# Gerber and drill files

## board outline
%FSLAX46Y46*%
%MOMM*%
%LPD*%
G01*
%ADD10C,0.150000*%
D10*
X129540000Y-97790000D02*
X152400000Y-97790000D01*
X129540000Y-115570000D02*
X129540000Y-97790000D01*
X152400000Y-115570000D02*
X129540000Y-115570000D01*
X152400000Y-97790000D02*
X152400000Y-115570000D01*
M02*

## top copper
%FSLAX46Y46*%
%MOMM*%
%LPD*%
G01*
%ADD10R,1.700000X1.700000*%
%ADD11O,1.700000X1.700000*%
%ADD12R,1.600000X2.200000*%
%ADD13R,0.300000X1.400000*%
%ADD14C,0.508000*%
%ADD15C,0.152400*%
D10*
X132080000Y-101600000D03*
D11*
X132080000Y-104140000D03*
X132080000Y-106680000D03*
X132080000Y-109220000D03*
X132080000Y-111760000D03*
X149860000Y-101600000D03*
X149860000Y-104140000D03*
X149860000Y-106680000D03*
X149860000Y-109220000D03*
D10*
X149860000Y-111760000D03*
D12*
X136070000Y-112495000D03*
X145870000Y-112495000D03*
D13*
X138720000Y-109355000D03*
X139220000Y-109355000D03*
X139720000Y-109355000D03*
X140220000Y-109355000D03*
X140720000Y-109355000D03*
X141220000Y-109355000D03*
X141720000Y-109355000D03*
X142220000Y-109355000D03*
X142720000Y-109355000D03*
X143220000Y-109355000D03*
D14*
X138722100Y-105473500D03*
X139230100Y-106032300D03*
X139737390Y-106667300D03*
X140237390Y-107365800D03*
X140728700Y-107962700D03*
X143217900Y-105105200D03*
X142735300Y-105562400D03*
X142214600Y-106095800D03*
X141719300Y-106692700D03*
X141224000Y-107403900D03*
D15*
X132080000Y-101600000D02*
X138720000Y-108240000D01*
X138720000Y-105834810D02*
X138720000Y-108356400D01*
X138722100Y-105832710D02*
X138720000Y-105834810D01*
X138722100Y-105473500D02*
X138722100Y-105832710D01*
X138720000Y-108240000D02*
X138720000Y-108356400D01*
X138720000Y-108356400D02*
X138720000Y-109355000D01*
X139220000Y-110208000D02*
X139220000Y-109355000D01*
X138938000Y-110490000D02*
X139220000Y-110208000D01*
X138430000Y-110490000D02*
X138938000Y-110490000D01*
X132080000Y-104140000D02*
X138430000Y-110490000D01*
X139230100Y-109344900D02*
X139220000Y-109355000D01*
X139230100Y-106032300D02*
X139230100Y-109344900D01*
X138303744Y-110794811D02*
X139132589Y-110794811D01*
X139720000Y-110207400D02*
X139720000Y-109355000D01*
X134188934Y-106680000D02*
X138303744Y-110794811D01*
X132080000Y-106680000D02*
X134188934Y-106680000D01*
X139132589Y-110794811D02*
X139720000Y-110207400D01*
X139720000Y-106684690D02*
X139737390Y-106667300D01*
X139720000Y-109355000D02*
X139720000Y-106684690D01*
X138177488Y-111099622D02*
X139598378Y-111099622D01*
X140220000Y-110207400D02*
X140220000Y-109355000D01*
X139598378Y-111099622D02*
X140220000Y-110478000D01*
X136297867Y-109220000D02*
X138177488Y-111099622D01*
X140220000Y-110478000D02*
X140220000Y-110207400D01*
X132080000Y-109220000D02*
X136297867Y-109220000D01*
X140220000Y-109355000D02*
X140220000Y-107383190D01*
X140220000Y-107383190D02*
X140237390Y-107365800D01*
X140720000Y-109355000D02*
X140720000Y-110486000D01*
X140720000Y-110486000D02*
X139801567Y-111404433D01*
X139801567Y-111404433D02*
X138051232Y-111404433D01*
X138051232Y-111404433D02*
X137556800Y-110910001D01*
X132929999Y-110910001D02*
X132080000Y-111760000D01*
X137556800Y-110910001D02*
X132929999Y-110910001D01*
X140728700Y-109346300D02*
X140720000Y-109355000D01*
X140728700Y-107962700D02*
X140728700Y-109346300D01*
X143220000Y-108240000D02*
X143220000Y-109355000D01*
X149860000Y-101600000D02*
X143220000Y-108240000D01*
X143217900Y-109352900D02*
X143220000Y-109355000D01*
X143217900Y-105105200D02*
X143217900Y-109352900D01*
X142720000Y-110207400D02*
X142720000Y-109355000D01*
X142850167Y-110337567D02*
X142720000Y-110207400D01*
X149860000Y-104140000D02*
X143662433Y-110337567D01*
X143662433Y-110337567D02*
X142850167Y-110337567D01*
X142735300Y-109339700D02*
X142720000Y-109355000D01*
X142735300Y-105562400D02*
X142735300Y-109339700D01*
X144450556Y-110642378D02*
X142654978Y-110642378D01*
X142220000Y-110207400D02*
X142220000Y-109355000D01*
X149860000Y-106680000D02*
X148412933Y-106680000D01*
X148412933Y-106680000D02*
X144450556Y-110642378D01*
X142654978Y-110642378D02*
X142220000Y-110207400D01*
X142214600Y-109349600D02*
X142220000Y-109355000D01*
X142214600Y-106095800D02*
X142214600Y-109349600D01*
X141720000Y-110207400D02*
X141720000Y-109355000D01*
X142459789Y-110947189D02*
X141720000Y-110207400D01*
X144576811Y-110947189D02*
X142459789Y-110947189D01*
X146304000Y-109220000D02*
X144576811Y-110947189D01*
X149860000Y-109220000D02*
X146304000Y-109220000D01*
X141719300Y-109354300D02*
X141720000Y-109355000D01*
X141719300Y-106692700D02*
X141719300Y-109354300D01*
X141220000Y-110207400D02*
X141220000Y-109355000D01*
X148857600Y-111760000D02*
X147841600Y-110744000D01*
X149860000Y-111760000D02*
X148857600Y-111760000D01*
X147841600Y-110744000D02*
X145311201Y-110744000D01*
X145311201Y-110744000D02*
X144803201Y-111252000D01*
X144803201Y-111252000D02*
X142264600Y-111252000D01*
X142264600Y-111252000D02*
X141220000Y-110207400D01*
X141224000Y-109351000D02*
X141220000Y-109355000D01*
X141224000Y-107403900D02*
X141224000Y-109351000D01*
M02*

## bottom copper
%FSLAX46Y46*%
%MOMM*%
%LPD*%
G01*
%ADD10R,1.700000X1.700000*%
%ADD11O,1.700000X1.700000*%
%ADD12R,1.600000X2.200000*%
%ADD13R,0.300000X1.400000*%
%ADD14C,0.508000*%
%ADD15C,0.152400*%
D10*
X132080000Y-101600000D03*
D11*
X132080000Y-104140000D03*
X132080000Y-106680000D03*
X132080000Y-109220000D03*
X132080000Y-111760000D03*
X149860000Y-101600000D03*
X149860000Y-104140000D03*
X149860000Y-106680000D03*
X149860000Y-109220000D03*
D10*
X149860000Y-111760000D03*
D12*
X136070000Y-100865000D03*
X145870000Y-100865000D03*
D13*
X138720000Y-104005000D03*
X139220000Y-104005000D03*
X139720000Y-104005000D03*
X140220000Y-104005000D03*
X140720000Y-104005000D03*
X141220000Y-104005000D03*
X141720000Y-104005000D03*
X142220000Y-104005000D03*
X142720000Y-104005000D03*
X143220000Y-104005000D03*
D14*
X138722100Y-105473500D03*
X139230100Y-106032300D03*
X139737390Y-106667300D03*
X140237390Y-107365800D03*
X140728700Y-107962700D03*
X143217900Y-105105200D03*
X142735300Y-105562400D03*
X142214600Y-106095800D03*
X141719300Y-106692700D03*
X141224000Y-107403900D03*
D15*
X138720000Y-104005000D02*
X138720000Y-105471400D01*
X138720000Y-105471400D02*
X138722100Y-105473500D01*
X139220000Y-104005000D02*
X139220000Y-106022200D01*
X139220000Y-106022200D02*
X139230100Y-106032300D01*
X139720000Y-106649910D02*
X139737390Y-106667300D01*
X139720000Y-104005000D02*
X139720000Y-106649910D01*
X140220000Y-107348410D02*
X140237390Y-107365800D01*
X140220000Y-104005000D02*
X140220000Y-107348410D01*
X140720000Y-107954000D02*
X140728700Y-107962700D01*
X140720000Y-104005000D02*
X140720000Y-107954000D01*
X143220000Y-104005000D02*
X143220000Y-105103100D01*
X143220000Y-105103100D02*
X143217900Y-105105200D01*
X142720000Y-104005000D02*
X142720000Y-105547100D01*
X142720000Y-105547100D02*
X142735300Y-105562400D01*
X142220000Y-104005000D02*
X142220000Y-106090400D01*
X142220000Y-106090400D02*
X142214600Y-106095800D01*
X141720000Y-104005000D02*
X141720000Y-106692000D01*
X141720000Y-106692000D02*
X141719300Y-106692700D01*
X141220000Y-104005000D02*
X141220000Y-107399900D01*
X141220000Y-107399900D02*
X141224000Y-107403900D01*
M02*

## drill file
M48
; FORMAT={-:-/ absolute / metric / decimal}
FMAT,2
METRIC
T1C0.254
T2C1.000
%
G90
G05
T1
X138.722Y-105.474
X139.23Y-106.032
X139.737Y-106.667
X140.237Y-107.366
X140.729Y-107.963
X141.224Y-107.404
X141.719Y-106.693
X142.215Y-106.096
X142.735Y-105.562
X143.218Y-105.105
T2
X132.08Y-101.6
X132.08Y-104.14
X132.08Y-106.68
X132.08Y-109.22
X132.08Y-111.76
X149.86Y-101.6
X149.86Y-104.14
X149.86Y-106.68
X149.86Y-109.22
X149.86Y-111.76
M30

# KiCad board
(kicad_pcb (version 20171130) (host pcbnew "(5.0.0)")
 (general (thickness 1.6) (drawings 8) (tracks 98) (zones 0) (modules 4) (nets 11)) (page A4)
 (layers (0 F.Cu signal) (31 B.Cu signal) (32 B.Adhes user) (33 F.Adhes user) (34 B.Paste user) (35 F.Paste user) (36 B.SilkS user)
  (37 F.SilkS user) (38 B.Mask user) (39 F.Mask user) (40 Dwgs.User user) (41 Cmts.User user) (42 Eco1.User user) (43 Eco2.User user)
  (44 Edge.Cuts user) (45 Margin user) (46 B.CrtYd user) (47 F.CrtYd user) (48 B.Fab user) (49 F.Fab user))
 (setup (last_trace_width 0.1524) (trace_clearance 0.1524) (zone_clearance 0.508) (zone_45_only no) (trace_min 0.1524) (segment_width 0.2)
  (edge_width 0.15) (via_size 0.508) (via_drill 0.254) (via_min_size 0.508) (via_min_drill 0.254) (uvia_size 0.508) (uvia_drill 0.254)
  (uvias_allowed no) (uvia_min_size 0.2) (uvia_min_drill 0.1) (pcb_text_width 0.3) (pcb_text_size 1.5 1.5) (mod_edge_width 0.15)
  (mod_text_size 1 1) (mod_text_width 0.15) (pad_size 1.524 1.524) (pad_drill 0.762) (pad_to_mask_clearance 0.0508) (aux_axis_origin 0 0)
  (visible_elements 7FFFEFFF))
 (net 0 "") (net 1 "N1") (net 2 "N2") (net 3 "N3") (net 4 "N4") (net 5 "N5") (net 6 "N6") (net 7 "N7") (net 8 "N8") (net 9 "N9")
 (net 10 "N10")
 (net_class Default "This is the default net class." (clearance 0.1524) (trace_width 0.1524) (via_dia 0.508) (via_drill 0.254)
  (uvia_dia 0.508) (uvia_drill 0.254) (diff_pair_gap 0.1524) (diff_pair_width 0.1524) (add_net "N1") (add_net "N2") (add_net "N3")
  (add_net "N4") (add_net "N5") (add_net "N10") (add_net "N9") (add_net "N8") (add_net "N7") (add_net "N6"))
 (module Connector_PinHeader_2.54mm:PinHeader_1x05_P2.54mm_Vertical (layer F.Cu) (at 132.08 101.6)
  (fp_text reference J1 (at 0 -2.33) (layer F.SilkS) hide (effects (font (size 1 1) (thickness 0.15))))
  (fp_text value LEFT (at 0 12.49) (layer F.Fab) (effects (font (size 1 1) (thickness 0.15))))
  (pad 1 thru_hole rect (at 0 0) (size 1.7 1.7) (drill 1) (layers *.Cu *.Mask) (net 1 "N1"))
  (pad 2 thru_hole oval (at 0 2.54) (size 1.7 1.7) (drill 1) (layers *.Cu *.Mask) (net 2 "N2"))
  (pad 3 thru_hole oval (at 0 5.08) (size 1.7 1.7) (drill 1) (layers *.Cu *.Mask) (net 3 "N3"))
  (pad 4 thru_hole oval (at 0 7.62) (size 1.7 1.7) (drill 1) (layers *.Cu *.Mask) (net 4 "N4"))
  (pad 5 thru_hole oval (at 0 10.16) (size 1.7 1.7) (drill 1) (layers *.Cu *.Mask) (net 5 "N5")))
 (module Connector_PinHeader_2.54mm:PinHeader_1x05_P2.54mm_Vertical (layer F.Cu) (at 149.86 111.76 180)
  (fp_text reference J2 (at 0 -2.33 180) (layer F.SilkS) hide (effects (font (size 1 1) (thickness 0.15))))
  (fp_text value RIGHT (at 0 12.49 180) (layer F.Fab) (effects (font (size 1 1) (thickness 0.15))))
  (pad 5 thru_hole oval (at 0 10.16 180) (size 1.7 1.7) (drill 1) (layers *.Cu *.Mask) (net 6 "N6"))
  (pad 4 thru_hole oval (at 0 7.62 180) (size 1.7 1.7) (drill 1) (layers *.Cu *.Mask) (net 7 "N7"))
  (pad 3 thru_hole oval (at 0 5.08 180) (size 1.7 1.7) (drill 1) (layers *.Cu *.Mask) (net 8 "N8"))
  (pad 2 thru_hole oval (at 0 2.54 180) (size 1.7 1.7) (drill 1) (layers *.Cu *.Mask) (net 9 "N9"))
  (pad 1 thru_hole rect (at 0 0 180) (size 1.7 1.7) (drill 1) (layers *.Cu *.Mask) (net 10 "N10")))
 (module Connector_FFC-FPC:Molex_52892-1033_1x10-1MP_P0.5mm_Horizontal (layer B.Cu) (at 140.97 102.235)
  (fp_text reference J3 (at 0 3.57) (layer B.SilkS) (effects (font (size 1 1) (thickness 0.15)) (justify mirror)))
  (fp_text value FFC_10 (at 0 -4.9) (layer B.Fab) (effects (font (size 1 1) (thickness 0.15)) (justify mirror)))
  (pad MP smd rect (at -4.9 -1.37) (size 1.6 2.2) (layers B.Cu B.Paste B.Mask))
  (pad MP smd rect (at 4.9 -1.37) (size 1.6 2.2) (layers B.Cu B.Paste B.Mask))
  (pad 1 smd rect (at -2.25 1.77) (size 0.3 1.4) (layers B.Cu B.Paste B.Mask) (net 1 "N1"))
  (pad 2 smd rect (at -1.75 1.77) (size 0.3 1.4) (layers B.Cu B.Paste B.Mask) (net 2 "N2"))
  (pad 3 smd rect (at -1.25 1.77) (size 0.3 1.4) (layers B.Cu B.Paste B.Mask) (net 3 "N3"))
  (pad 4 smd rect (at -0.75 1.77) (size 0.3 1.4) (layers B.Cu B.Paste B.Mask) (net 4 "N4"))
  (pad 5 smd rect (at -0.25 1.77) (size 0.3 1.4) (layers B.Cu B.Paste B.Mask) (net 5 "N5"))
  (pad 6 smd rect (at 0.25 1.77) (size 0.3 1.4) (layers B.Cu B.Paste B.Mask) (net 10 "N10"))
  (pad 7 smd rect (at 0.75 1.77) (size 0.3 1.4) (layers B.Cu B.Paste B.Mask) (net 9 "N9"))
  (pad 8 smd rect (at 1.25 1.77) (size 0.3 1.4) (layers B.Cu B.Paste B.Mask) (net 8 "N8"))
  (pad 9 smd rect (at 1.75 1.77) (size 0.3 1.4) (layers B.Cu B.Paste B.Mask) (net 7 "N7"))
  (pad 10 smd rect (at 2.25 1.77) (size 0.3 1.4) (layers B.Cu B.Paste B.Mask) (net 6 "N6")))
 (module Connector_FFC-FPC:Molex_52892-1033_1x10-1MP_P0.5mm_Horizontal (layer F.Cu) (at 140.97 111.125)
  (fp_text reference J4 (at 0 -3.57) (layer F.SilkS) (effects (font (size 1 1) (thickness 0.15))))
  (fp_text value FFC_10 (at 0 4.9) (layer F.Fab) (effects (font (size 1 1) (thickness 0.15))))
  (pad MP smd rect (at -4.9 1.37) (size 1.6 2.2) (layers F.Cu F.Paste F.Mask))
  (pad MP smd rect (at 4.9 1.37) (size 1.6 2.2) (layers F.Cu F.Paste F.Mask))
  (pad 1 smd rect (at -2.25 -1.77) (size 0.3 1.4) (layers F.Cu F.Paste F.Mask) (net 1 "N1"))
  (pad 2 smd rect (at -1.75 -1.77) (size 0.3 1.4) (layers F.Cu F.Paste F.Mask) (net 2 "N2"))
  (pad 3 smd rect (at -1.25 -1.77) (size 0.3 1.4) (layers F.Cu F.Paste F.Mask) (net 3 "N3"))
  (pad 4 smd rect (at -0.75 -1.77) (size 0.3 1.4) (layers F.Cu F.Paste F.Mask) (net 4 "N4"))
  (pad 5 smd rect (at -0.25 -1.77) (size 0.3 1.4) (layers F.Cu F.Paste F.Mask) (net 5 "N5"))
  (pad 6 smd rect (at 0.25 -1.77) (size 0.3 1.4) (layers F.Cu F.Paste F.Mask) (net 10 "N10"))
  (pad 7 smd rect (at 0.75 -1.77) (size 0.3 1.4) (layers F.Cu F.Paste F.Mask) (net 9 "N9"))
  (pad 8 smd rect (at 1.25 -1.77) (size 0.3 1.4) (layers F.Cu F.Paste F.Mask) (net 8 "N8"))
  (pad 9 smd rect (at 1.75 -1.77) (size 0.3 1.4) (layers F.Cu F.Paste F.Mask) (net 7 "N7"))
  (pad 10 smd rect (at 2.25 -1.77) (size 0.3 1.4) (layers F.Cu F.Paste F.Mask) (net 6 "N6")))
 (gr_line (start 129.54 97.79) (end 152.4 97.79) (layer Edge.Cuts) (width 0.15))
 (gr_line (start 129.54 115.57) (end 129.54 97.79) (layer Edge.Cuts) (width 0.15))
 (gr_line (start 152.4 115.57) (end 129.54 115.57) (layer Edge.Cuts) (width 0.15))
 (gr_line (start 152.4 97.79) (end 152.4 115.57) (layer Edge.Cuts) (width 0.15))
 (segment (start 132.08 101.6) (end 138.72 108.24) (width 0.1524) (layer F.Cu) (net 1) (status 10))
 (via (at 138.7221 105.4735) (size 0.508) (drill 0.254) (layers F.Cu B.Cu) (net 1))
 (segment (start 138.72 104.005) (end 138.72 105.4714) (width 0.1524) (layer B.Cu) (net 1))
 (segment (start 138.72 105.4714) (end 138.7221 105.4735) (width 0.1524) (layer B.Cu) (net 1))
 (segment (start 138.72 105.83481) (end 138.72 108.3564) (width 0.1524) (layer F.Cu) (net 1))
 (segment (start 138.7221 105.83271) (end 138.72 105.83481) (width 0.1524) (layer F.Cu) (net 1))
 (segment (start 138.7221 105.4735) (end 138.7221 105.83271) (width 0.1524) (layer F.Cu) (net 1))
 (segment (start 138.72 108.24) (end 138.72 108.3564) (width 0.1524) (layer F.Cu) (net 1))
 (segment (start 138.72 108.3564) (end 138.72 109.355) (width 0.1524) (layer F.Cu) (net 1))
 (segment (start 139.22 110.208) (end 139.22 109.355) (width 0.1524) (layer F.Cu) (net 2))
 (segment (start 138.938 110.49) (end 139.22 110.208) (width 0.1524) (layer F.Cu) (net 2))
 (segment (start 138.43 110.49) (end 138.938 110.49) (width 0.1524) (layer F.Cu) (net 2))
 (segment (start 132.08 104.14) (end 138.43 110.49) (width 0.1524) (layer F.Cu) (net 2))
 (via (at 139.2301 106.0323) (size 0.508) (drill 0.254) (layers F.Cu B.Cu) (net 2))
 (segment (start 139.22 104.005) (end 139.22 106.0222) (width 0.1524) (layer B.Cu) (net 2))
 (segment (start 139.22 106.0222) (end 139.2301 106.0323) (width 0.1524) (layer B.Cu) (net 2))
 (segment (start 139.2301 109.3449) (end 139.22 109.355) (width 0.1524) (layer F.Cu) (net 2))
 (segment (start 139.2301 106.0323) (end 139.2301 109.3449) (width 0.1524) (layer F.Cu) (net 2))
 (segment (start 138.303744 110.794811) (end 139.132589 110.794811) (width 0.1524) (layer F.Cu) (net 3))
 (segment (start 139.72 110.2074) (end 139.72 109.355) (width 0.1524) (layer F.Cu) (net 3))
 (segment (start 134.188934 106.68) (end 138.303744 110.794811) (width 0.1524) (layer F.Cu) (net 3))
 (segment (start 132.08 106.68) (end 134.188934 106.68) (width 0.1524) (layer F.Cu) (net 3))
 (segment (start 139.132589 110.794811) (end 139.72 110.2074) (width 0.1524) (layer F.Cu) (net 3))
 (segment (start 139.72 106.64991) (end 139.73739 106.6673) (width 0.1524) (layer B.Cu) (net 3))
 (segment (start 139.72 106.68469) (end 139.73739 106.6673) (width 0.1524) (layer F.Cu) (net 3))
 (segment (start 139.72 104.005) (end 139.72 106.64991) (width 0.1524) (layer B.Cu) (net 3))
 (segment (start 139.72 109.355) (end 139.72 106.68469) (width 0.1524) (layer F.Cu) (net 3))
 (via (at 139.73739 106.6673) (size 0.508) (drill 0.254) (layers F.Cu B.Cu) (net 3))
 (segment (start 138.177488 111.099622) (end 139.598378 111.099622) (width 0.1524) (layer F.Cu) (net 4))
 (segment (start 140.22 110.2074) (end 140.22 109.355) (width 0.1524) (layer F.Cu) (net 4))
 (segment (start 139.598378 111.099622) (end 140.22 110.478) (width 0.1524) (layer F.Cu) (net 4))
 (segment (start 136.297867 109.22) (end 138.177488 111.099622) (width 0.1524) (layer F.Cu) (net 4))
 (segment (start 140.22 110.478) (end 140.22 110.2074) (width 0.1524) (layer F.Cu) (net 4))
 (segment (start 132.08 109.22) (end 136.297867 109.22) (width 0.1524) (layer F.Cu) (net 4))
 (segment (start 140.22 109.355) (end 140.22 107.38319) (width 0.1524) (layer F.Cu) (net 4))
 (segment (start 140.22 107.38319) (end 140.23739 107.3658) (width 0.1524) (layer F.Cu) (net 4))
 (segment (start 140.22 107.34841) (end 140.23739 107.3658) (width 0.1524) (layer B.Cu) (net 4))
 (segment (start 140.22 104.005) (end 140.22 107.34841) (width 0.1524) (layer B.Cu) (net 4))
 (via (at 140.23739 107.3658) (size 0.508) (drill 0.254) (layers F.Cu B.Cu) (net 4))
 (segment (start 140.72 109.355) (end 140.72 110.486) (width 0.1524) (layer F.Cu) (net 5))
 (segment (start 140.72 110.486) (end 139.801567 111.404433) (width 0.1524) (layer F.Cu) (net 5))
 (segment (start 139.801567 111.404433) (end 138.051232 111.404433) (width 0.1524) (layer F.Cu) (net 5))
 (segment (start 138.051232 111.404433) (end 137.5568 110.910001) (width 0.1524) (layer F.Cu) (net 5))
 (segment (start 132.929999 110.910001) (end 132.08 111.76) (width 0.1524) (layer F.Cu) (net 5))
 (segment (start 137.5568 110.910001) (end 132.929999 110.910001) (width 0.1524) (layer F.Cu) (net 5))
 (via (at 140.7287 107.9627) (size 0.508) (drill 0.254) (layers F.Cu B.Cu) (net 5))
 (segment (start 140.72 107.954) (end 140.7287 107.9627) (width 0.1524) (layer B.Cu) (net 5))
 (segment (start 140.72 104.005) (end 140.72 107.954) (width 0.1524) (layer B.Cu) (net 5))
 (segment (start 140.7287 109.3463) (end 140.72 109.355) (width 0.1524) (layer F.Cu) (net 5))
 (segment (start 140.7287 107.9627) (end 140.7287 109.3463) (width 0.1524) (layer F.Cu) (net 5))
 (segment (start 143.22 108.24) (end 143.22 109.355) (width 0.1524) (layer F.Cu) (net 6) (status 20))
 (segment (start 149.86 101.6) (end 143.22 108.24) (width 0.1524) (layer F.Cu) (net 6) (status 10))
 (via (at 143.2179 105.1052) (size 0.508) (drill 0.254) (layers F.Cu B.Cu) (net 6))
 (segment (start 143.22 104.005) (end 143.22 105.1031) (width 0.1524) (layer B.Cu) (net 6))
 (segment (start 143.22 105.1031) (end 143.2179 105.1052) (width 0.1524) (layer B.Cu) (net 6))
 (segment (start 143.2179 109.3529) (end 143.22 109.355) (width 0.1524) (layer F.Cu) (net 6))
 (segment (start 143.2179 105.1052) (end 143.2179 109.3529) (width 0.1524) (layer F.Cu) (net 6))
 (segment (start 142.72 110.2074) (end 142.72 109.355) (width 0.1524) (layer F.Cu) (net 7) (status 20))
 (segment (start 142.850167 110.337567) (end 142.72 110.2074) (width 0.1524) (layer F.Cu) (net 7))
 (segment (start 149.86 104.14) (end 143.662433 110.337567) (width 0.1524) (layer F.Cu) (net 7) (status 10))
 (segment (start 143.662433 110.337567) (end 142.850167 110.337567) (width 0.1524) (layer F.Cu) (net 7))
 (via (at 142.7353 105.5624) (size 0.508) (drill 0.254) (layers F.Cu B.Cu) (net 7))
 (segment (start 142.72 104.005) (end 142.72 105.5471) (width 0.1524) (layer B.Cu) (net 7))
 (segment (start 142.72 105.5471) (end 142.7353 105.5624) (width 0.1524) (layer B.Cu) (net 7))
 (segment (start 142.7353 109.3397) (end 142.72 109.355) (width 0.1524) (layer F.Cu) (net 7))
 (segment (start 142.7353 105.5624) (end 142.7353 109.3397) (width 0.1524) (layer F.Cu) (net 7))
 (segment (start 144.450556 110.642378) (end 142.654978 110.642378) (width 0.1524) (layer F.Cu) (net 8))
 (segment (start 142.22 110.2074) (end 142.22 109.355) (width 0.1524) (layer F.Cu) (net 8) (status 20))
 (segment (start 149.86 106.68) (end 148.412933 106.68) (width 0.1524) (layer F.Cu) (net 8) (status 10))
 (segment (start 148.412933 106.68) (end 144.450556 110.642378) (width 0.1524) (layer F.Cu) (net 8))
 (segment (start 142.654978 110.642378) (end 142.22 110.2074) (width 0.1524) (layer F.Cu) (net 8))
 (via (at 142.2146 106.0958) (size 0.508) (drill 0.254) (layers F.Cu B.Cu) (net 8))
 (segment (start 142.22 104.005) (end 142.22 106.0904) (width 0.1524) (layer B.Cu) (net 8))
 (segment (start 142.22 106.0904) (end 142.2146 106.0958) (width 0.1524) (layer B.Cu) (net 8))
 (segment (start 142.2146 109.3496) (end 142.22 109.355) (width 0.1524) (layer F.Cu) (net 8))
 (segment (start 142.2146 106.0958) (end 142.2146 109.3496) (width 0.1524) (layer F.Cu) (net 8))
 (segment (start 141.72 110.2074) (end 141.72 109.355) (width 0.1524) (layer F.Cu) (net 9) (status 20))
 (segment (start 142.459789 110.947189) (end 141.72 110.2074) (width 0.1524) (layer F.Cu) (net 9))
 (segment (start 144.576811 110.947189) (end 142.459789 110.947189) (width 0.1524) (layer F.Cu) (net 9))
 (segment (start 146.304 109.22) (end 144.576811 110.947189) (width 0.1524) (layer F.Cu) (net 9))
 (segment (start 149.86 109.22) (end 146.304 109.22) (width 0.1524) (layer F.Cu) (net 9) (status 10))
 (via (at 141.7193 106.6927) (size 0.508) (drill 0.254) (layers F.Cu B.Cu) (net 9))
 (segment (start 141.72 104.005) (end 141.72 106.692) (width 0.1524) (layer B.Cu) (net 9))
 (segment (start 141.72 106.692) (end 141.7193 106.6927) (width 0.1524) (layer B.Cu) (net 9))
 (segment (start 141.7193 109.3543) (end 141.72 109.355) (width 0.1524) (layer F.Cu) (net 9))
 (segment (start 141.7193 106.6927) (end 141.7193 109.3543) (width 0.1524) (layer F.Cu) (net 9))
 (segment (start 141.22 110.2074) (end 141.22 109.355) (width 0.1524) (layer F.Cu) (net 10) (status 20))
 (segment (start 148.8576 111.76) (end 147.8416 110.744) (width 0.1524) (layer F.Cu) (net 10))
 (segment (start 149.86 111.76) (end 148.8576 111.76) (width 0.1524) (layer F.Cu) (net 10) (status 10))
 (segment (start 147.8416 110.744) (end 145.311201 110.744) (width 0.1524) (layer F.Cu) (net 10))
 (segment (start 145.311201 110.744) (end 144.803201 111.252) (width 0.1524) (layer F.Cu) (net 10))
 (segment (start 144.803201 111.252) (end 142.2646 111.252) (width 0.1524) (layer F.Cu) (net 10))
 (segment (start 142.2646 111.252) (end 141.22 110.2074) (width 0.1524) (layer F.Cu) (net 10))
 (via (at 141.224 107.4039) (size 0.508) (drill 0.254) (layers F.Cu B.Cu) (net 10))
 (segment (start 141.22 104.005) (end 141.22 107.3999) (width 0.1524) (layer B.Cu) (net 10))
 (segment (start 141.22 107.3999) (end 141.224 107.4039) (width 0.1524) (layer B.Cu) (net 10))
 (segment (start 141.224 109.351) (end 141.22 109.355) (width 0.1524) (layer F.Cu) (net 10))
 (segment (start 141.224 107.4039) (end 141.224 109.351) (width 0.1524) (layer F.Cu) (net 10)))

